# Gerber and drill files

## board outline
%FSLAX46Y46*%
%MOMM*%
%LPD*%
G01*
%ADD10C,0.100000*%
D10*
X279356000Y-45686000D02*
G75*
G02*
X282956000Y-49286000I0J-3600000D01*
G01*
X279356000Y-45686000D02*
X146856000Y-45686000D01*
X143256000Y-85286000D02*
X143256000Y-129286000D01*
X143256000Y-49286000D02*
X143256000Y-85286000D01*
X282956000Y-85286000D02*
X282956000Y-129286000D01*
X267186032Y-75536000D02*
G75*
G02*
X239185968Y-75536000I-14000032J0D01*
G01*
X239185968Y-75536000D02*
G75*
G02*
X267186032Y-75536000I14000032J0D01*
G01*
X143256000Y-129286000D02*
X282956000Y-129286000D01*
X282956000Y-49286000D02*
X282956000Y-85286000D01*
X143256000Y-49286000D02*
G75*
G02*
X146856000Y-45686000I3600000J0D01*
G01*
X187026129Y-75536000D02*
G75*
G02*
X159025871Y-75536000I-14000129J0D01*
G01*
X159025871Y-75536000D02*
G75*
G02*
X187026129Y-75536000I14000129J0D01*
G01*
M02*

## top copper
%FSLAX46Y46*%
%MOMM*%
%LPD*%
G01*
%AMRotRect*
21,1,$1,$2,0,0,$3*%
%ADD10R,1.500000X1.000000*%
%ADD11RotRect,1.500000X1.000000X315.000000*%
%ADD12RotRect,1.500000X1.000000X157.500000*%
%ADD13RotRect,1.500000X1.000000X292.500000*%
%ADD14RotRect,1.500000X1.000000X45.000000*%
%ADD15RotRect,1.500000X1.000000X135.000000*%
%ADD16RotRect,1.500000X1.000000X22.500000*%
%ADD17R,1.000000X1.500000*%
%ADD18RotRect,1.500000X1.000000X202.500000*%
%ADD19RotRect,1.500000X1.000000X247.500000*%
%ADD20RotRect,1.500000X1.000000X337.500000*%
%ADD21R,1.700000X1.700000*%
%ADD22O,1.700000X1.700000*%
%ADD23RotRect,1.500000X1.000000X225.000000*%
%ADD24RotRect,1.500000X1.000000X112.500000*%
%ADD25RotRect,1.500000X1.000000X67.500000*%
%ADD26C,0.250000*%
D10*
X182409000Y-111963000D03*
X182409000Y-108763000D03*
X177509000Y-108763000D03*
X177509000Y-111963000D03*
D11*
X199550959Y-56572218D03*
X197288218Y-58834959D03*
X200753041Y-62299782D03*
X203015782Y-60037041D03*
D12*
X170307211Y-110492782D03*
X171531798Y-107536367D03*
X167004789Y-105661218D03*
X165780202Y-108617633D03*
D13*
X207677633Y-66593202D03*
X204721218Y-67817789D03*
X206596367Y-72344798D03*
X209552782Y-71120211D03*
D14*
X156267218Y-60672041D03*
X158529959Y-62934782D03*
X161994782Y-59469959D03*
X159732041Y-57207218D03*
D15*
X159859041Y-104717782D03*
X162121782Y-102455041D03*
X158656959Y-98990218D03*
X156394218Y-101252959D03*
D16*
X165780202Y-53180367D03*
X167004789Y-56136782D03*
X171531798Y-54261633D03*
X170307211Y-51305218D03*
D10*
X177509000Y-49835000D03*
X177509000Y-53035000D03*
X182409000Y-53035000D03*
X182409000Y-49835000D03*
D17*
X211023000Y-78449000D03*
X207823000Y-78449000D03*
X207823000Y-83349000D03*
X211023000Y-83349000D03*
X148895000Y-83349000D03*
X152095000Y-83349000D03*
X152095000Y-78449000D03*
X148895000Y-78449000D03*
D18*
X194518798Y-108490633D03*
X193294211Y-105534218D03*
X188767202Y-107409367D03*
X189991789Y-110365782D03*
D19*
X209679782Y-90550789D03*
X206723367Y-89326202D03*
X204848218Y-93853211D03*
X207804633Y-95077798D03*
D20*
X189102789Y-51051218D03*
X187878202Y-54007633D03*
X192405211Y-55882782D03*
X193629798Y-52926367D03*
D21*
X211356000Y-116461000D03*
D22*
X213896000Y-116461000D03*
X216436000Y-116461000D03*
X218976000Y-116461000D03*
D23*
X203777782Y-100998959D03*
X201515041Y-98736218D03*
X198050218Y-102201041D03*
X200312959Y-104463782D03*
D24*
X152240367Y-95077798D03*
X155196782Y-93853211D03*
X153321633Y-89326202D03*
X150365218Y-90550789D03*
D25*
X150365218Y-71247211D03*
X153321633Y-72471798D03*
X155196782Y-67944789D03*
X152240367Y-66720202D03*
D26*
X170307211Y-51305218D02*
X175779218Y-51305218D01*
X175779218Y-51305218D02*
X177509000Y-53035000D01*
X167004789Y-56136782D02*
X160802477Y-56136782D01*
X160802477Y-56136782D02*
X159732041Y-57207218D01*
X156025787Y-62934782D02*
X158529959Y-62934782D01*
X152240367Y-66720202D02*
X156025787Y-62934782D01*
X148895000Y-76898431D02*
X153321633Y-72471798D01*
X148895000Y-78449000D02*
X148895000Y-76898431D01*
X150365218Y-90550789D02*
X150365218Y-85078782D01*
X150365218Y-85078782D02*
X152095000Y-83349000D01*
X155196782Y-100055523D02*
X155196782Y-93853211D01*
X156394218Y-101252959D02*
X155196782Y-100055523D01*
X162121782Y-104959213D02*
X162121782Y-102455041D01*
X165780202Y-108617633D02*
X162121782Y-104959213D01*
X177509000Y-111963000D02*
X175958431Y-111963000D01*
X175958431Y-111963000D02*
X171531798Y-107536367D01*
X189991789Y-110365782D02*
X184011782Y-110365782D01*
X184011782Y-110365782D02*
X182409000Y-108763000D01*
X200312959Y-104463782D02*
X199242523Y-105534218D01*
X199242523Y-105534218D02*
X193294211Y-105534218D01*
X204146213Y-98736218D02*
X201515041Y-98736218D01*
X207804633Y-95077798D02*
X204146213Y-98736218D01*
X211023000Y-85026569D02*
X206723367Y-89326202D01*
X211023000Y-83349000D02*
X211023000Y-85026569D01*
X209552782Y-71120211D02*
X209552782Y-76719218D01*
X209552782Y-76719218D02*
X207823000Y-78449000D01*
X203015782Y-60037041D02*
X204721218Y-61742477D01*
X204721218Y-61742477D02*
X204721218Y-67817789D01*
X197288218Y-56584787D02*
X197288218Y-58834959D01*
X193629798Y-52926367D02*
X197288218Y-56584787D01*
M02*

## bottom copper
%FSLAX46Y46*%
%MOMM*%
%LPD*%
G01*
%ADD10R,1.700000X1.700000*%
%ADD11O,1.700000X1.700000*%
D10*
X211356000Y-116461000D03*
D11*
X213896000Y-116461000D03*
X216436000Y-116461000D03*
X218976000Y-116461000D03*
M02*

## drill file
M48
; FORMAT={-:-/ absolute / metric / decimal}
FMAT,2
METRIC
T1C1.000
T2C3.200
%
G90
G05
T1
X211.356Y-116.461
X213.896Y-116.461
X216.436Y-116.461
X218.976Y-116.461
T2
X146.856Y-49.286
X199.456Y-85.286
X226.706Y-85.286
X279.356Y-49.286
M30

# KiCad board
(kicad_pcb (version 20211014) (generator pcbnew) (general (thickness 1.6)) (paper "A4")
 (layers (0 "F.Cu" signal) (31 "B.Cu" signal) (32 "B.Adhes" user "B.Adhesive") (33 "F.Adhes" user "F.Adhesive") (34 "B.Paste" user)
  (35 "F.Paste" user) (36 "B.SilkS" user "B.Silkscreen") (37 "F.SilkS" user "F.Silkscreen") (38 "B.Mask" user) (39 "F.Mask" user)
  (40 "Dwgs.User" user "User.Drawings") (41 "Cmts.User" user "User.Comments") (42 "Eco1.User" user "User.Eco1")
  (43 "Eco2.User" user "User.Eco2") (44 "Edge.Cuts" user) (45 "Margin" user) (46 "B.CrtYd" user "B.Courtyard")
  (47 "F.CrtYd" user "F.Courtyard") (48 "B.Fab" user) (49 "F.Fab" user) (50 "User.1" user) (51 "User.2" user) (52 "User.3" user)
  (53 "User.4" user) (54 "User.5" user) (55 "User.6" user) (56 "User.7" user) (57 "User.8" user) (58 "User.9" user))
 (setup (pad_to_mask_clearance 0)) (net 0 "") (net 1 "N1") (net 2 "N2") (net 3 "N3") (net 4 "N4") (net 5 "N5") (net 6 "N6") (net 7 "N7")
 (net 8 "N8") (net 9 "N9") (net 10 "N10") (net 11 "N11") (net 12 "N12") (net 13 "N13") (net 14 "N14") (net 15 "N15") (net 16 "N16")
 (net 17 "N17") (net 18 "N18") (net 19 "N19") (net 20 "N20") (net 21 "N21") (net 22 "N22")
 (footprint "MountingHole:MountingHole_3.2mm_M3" (layer "F.Cu") (at 226.706 85.286)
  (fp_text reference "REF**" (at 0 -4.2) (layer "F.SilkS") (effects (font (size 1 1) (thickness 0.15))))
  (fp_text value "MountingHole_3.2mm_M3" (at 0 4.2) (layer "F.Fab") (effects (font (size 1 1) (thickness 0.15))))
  (pad "" np_thru_hole circle locked (at 0 0) (size 3.2 3.2) (drill 3.2) (layers *.Cu *.Mask)))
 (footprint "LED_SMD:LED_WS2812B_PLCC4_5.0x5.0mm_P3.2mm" (layer "F.Cu") (at 179.959 110.363 180)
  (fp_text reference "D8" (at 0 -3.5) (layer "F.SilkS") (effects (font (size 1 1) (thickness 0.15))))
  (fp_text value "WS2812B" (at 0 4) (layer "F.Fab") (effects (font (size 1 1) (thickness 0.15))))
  (pad "1" smd rect locked (at -2.45 -1.6 180) (size 1.5 1) (layers "F.Cu" "F.Paste" "F.Mask") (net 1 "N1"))
  (pad "2" smd rect locked (at -2.45 1.6 180) (size 1.5 1) (layers "F.Cu" "F.Paste" "F.Mask") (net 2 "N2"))
  (pad "3" smd rect locked (at 2.45 1.6 180) (size 1.5 1) (layers "F.Cu" "F.Paste" "F.Mask") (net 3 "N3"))
  (pad "4" smd rect locked (at 2.45 -1.6 180) (size 1.5 1) (layers "F.Cu" "F.Paste" "F.Mask") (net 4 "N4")))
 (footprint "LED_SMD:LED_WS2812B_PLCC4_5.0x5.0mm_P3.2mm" (layer "F.Cu") (at 200.152 59.436 -45)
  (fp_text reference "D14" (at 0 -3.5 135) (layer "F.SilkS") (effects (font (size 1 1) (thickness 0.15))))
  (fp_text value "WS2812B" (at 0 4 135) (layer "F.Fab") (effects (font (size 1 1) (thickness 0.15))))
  (pad "1" smd rect locked (at -2.45 -1.6 315) (size 1.5 1) (layers "F.Cu" "F.Paste" "F.Mask") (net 1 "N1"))
  (pad "2" smd rect locked (at -2.45 1.6 315) (size 1.5 1) (layers "F.Cu" "F.Paste" "F.Mask") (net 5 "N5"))
  (pad "3" smd rect locked (at 2.45 1.6 315) (size 1.5 1) (layers "F.Cu" "F.Paste" "F.Mask") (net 3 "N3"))
  (pad "4" smd rect locked (at 2.45 -1.6 315) (size 1.5 1) (layers "F.Cu" "F.Paste" "F.Mask") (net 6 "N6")))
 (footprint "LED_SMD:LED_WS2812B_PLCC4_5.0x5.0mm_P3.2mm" (layer "F.Cu") (at 168.656 108.077 157.5)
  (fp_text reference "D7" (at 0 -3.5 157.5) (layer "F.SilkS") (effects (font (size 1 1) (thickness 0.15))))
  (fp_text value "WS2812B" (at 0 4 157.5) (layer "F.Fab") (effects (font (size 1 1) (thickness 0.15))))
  (pad "1" smd rect locked (at -2.45 -1.6 157.5) (size 1.5 1) (layers "F.Cu" "F.Paste" "F.Mask") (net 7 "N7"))
  (pad "2" smd rect locked (at -2.45 1.6 157.5) (size 1.5 1) (layers "F.Cu" "F.Paste" "F.Mask") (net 4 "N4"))
  (pad "3" smd rect locked (at 2.45 1.6 157.5) (size 1.5 1) (layers "F.Cu" "F.Paste" "F.Mask") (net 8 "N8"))
  (pad "4" smd rect locked (at 2.45 -1.6 157.5) (size 1.5 1) (layers "F.Cu" "F.Paste" "F.Mask") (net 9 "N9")))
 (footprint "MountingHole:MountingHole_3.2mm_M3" (layer "F.Cu") (at 279.356 49.286)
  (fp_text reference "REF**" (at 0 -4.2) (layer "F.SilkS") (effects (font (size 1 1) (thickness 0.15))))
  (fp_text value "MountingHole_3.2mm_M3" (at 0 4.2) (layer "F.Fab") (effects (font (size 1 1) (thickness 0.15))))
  (pad "" np_thru_hole circle locked (at 0 0) (size 3.2 3.2) (drill 3.2) (layers *.Cu *.Mask)))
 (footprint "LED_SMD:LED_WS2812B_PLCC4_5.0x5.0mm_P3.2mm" (layer "F.Cu") (at 207.137 69.469 -67.5)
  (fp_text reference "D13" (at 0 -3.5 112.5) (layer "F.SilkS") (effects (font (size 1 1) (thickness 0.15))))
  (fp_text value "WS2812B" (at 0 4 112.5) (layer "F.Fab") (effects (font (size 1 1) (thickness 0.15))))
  (pad "1" smd rect locked (at -2.45 -1.6 292.5) (size 1.5 1) (layers "F.Cu" "F.Paste" "F.Mask") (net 1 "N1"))
  (pad "2" smd rect locked (at -2.45 1.6 292.5) (size 1.5 1) (layers "F.Cu" "F.Paste" "F.Mask") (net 6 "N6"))
  (pad "3" smd rect locked (at 2.45 1.6 292.5) (size 1.5 1) (layers "F.Cu" "F.Paste" "F.Mask") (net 3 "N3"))
  (pad "4" smd rect locked (at 2.45 -1.6 292.5) (size 1.5 1) (layers "F.Cu" "F.Paste" "F.Mask") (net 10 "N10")))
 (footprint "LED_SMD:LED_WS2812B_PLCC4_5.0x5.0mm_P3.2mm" (layer "F.Cu") (at 159.131 60.071 45)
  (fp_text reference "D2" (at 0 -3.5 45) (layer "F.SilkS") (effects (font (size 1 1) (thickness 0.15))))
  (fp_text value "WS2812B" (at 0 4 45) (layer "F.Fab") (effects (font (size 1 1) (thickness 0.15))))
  (pad "1" smd rect locked (at -2.45 -1.6 45) (size 1.5 1) (layers "F.Cu" "F.Paste" "F.Mask") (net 7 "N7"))
  (pad "2" smd rect locked (at -2.45 1.6 45) (size 1.5 1) (layers "F.Cu" "F.Paste" "F.Mask") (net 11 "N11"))
  (pad "3" smd rect locked (at 2.45 1.6 45) (size 1.5 1) (layers "F.Cu" "F.Paste" "F.Mask") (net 8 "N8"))
  (pad "4" smd rect locked (at 2.45 -1.6 45) (size 1.5 1) (layers "F.Cu" "F.Paste" "F.Mask") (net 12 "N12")))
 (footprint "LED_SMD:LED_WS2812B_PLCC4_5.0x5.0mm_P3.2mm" (layer "F.Cu") (at 159.258 101.854 135)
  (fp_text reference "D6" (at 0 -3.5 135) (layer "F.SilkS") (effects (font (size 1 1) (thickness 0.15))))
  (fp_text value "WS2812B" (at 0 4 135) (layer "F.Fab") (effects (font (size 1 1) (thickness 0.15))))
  (pad "1" smd rect locked (at -2.45 -1.6 135) (size 1.5 1) (layers "F.Cu" "F.Paste" "F.Mask") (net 7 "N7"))
  (pad "2" smd rect locked (at -2.45 1.6 135) (size 1.5 1) (layers "F.Cu" "F.Paste" "F.Mask") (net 9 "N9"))
  (pad "3" smd rect locked (at 2.45 1.6 135) (size 1.5 1) (layers "F.Cu" "F.Paste" "F.Mask") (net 8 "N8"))
  (pad "4" smd rect locked (at 2.45 -1.6 135) (size 1.5 1) (layers "F.Cu" "F.Paste" "F.Mask") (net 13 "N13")))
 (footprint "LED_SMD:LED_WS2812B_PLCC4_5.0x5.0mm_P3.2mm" (layer "F.Cu") (at 168.656 53.721 22.5)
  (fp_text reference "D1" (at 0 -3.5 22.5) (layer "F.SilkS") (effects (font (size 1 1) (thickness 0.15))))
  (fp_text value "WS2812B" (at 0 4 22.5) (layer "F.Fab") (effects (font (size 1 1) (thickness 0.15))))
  (pad "1" smd rect locked (at -2.45 -1.6 22.5) (size 1.5 1) (layers "F.Cu" "F.Paste" "F.Mask") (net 7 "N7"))
  (pad "2" smd rect locked (at -2.45 1.6 22.5) (size 1.5 1) (layers "F.Cu" "F.Paste" "F.Mask") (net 12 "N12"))
  (pad "3" smd rect locked (at 2.45 1.6 22.5) (size 1.5 1) (layers "F.Cu" "F.Paste" "F.Mask") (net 8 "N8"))
  (pad "4" smd rect locked (at 2.45 -1.6 22.5) (size 1.5 1) (layers "F.Cu" "F.Paste" "F.Mask") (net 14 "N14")))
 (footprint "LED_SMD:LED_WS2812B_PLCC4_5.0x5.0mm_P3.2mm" (layer "F.Cu") (at 179.959 51.435)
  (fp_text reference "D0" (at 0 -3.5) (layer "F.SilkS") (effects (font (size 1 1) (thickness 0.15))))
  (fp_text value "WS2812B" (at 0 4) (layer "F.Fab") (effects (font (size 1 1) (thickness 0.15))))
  (pad "1" smd rect locked (at -2.45 -1.6) (size 1.5 1) (layers "F.Cu" "F.Paste" "F.Mask") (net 7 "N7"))
  (pad "2" smd rect locked (at -2.45 1.6) (size 1.5 1) (layers "F.Cu" "F.Paste" "F.Mask") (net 14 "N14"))
  (pad "3" smd rect locked (at 2.45 1.6) (size 1.5 1) (layers "F.Cu" "F.Paste" "F.Mask") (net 8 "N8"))
  (pad "4" smd rect locked (at 2.45 -1.6) (size 1.5 1) (layers "F.Cu" "F.Paste" "F.Mask") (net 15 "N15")))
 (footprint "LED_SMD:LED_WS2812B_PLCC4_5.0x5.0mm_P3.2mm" (layer "F.Cu") (at 209.423 80.899 -90)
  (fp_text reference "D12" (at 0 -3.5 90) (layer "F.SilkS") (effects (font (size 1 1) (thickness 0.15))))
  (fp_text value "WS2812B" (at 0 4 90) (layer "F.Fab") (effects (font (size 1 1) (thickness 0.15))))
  (pad "1" smd rect locked (at -2.45 -1.6 270) (size 1.5 1) (layers "F.Cu" "F.Paste" "F.Mask") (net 1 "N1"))
  (pad "2" smd rect locked (at -2.45 1.6 270) (size 1.5 1) (layers "F.Cu" "F.Paste" "F.Mask") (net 10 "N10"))
  (pad "3" smd rect locked (at 2.45 1.6 270) (size 1.5 1) (layers "F.Cu" "F.Paste" "F.Mask") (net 3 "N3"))
  (pad "4" smd rect locked (at 2.45 -1.6 270) (size 1.5 1) (layers "F.Cu" "F.Paste" "F.Mask") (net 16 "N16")))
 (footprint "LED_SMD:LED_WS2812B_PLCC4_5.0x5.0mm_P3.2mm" (layer "F.Cu") (at 150.495 80.899 90)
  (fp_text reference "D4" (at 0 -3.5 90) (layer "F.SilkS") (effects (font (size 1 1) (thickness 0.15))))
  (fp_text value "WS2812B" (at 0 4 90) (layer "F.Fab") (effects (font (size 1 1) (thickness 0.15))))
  (pad "1" smd rect locked (at -2.45 -1.6 90) (size 1.5 1) (layers "F.Cu" "F.Paste" "F.Mask") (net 7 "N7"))
  (pad "2" smd rect locked (at -2.45 1.6 90) (size 1.5 1) (layers "F.Cu" "F.Paste" "F.Mask") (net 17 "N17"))
  (pad "3" smd rect locked (at 2.45 1.6 90) (size 1.5 1) (layers "F.Cu" "F.Paste" "F.Mask") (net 8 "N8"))
  (pad "4" smd rect locked (at 2.45 -1.6 90) (size 1.5 1) (layers "F.Cu" "F.Paste" "F.Mask") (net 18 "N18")))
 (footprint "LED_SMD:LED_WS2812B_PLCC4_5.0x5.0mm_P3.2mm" (layer "F.Cu") (at 191.643 107.95 -157.5)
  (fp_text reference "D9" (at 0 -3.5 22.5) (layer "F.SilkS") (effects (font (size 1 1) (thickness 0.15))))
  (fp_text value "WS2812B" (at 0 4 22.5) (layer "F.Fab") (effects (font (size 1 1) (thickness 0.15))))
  (pad "1" smd rect locked (at -2.45 -1.6 202.5) (size 1.5 1) (layers "F.Cu" "F.Paste" "F.Mask") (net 1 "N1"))
  (pad "2" smd rect locked (at -2.45 1.6 202.5) (size 1.5 1) (layers "F.Cu" "F.Paste" "F.Mask") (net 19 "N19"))
  (pad "3" smd rect locked (at 2.45 1.6 202.5) (size 1.5 1) (layers "F.Cu" "F.Paste" "F.Mask") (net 3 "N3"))
  (pad "4" smd rect locked (at 2.45 -1.6 202.5) (size 1.5 1) (layers "F.Cu" "F.Paste" "F.Mask") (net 2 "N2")))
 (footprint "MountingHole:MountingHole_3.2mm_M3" (layer "F.Cu") (at 146.856 49.286)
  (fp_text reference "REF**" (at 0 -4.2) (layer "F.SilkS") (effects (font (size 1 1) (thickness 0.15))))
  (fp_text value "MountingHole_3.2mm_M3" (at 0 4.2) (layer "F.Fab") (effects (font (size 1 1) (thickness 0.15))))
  (pad "" np_thru_hole circle locked (at 0 0) (size 3.2 3.2) (drill 3.2) (layers *.Cu *.Mask)))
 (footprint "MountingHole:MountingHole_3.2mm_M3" (layer "F.Cu") (at 199.456 85.286)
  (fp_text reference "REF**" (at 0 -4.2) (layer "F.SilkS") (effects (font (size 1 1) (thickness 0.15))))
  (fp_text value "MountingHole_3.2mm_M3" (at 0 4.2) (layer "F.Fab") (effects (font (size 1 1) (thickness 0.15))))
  (pad "" np_thru_hole circle locked (at 0 0) (size 3.2 3.2) (drill 3.2) (layers *.Cu *.Mask)))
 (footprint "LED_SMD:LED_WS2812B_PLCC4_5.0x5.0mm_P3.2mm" (layer "F.Cu") (at 207.264 92.202 -112.5)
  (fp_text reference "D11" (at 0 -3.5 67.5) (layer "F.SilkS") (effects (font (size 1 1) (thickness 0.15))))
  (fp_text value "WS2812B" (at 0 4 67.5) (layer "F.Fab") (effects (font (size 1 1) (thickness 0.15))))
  (pad "1" smd rect locked (at -2.45 -1.6 247.5) (size 1.5 1) (layers "F.Cu" "F.Paste" "F.Mask") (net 1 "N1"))
  (pad "2" smd rect locked (at -2.45 1.6 247.5) (size 1.5 1) (layers "F.Cu" "F.Paste" "F.Mask") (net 16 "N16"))
  (pad "3" smd rect locked (at 2.45 1.6 247.5) (size 1.5 1) (layers "F.Cu" "F.Paste" "F.Mask") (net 3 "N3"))
  (pad "4" smd rect locked (at 2.45 -1.6 247.5) (size 1.5 1) (layers "F.Cu" "F.Paste" "F.Mask") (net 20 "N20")))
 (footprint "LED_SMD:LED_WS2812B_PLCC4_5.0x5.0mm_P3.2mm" (layer "F.Cu") (at 190.754 53.467 -22.5)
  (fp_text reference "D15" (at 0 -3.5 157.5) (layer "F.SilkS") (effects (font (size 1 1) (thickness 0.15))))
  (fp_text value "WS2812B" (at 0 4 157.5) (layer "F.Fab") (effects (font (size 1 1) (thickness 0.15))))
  (pad "1" smd rect locked (at -2.45 -1.6 337.5) (size 1.5 1) (layers "F.Cu" "F.Paste" "F.Mask") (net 1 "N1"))
  (pad "2" smd rect locked (at -2.45 1.6 337.5) (size 1.5 1) (layers "F.Cu" "F.Paste" "F.Mask") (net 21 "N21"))
  (pad "3" smd rect locked (at 2.45 1.6 337.5) (size 1.5 1) (layers "F.Cu" "F.Paste" "F.Mask") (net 3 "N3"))
  (pad "4" smd rect locked (at 2.45 -1.6 337.5) (size 1.5 1) (layers "F.Cu" "F.Paste" "F.Mask") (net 5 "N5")))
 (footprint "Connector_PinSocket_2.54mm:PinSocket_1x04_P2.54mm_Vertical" (layer "F.Cu") (at 211.356 116.461 90)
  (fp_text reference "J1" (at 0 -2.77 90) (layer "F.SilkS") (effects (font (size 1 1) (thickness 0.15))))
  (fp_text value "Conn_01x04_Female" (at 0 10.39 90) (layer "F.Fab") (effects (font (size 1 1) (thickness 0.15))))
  (pad "1" thru_hole rect locked (at 0 0 90) (size 1.7 1.7) (drill 1) (layers *.Cu *.Mask) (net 8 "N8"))
  (pad "2" thru_hole oval locked (at 0 2.54 90) (size 1.7 1.7) (drill 1) (layers *.Cu *.Mask) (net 7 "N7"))
  (pad "3" thru_hole oval locked (at 0 5.08 90) (size 1.7 1.7) (drill 1) (layers *.Cu *.Mask) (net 15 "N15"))
  (pad "4" thru_hole oval locked (at 0 7.62 90) (size 1.7 1.7) (drill 1) (layers *.Cu *.Mask) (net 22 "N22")))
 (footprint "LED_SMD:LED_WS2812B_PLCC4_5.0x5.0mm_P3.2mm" (layer "F.Cu") (at 200.914 101.6 -135)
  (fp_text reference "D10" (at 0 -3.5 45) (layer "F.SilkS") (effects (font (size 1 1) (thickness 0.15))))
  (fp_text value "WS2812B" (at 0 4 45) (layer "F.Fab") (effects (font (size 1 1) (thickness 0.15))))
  (pad "1" smd rect locked (at -2.45 -1.6 225) (size 1.5 1) (layers "F.Cu" "F.Paste" "F.Mask") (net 1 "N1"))
  (pad "2" smd rect locked (at -2.45 1.6 225) (size 1.5 1) (layers "F.Cu" "F.Paste" "F.Mask") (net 20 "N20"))
  (pad "3" smd rect locked (at 2.45 1.6 225) (size 1.5 1) (layers "F.Cu" "F.Paste" "F.Mask") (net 3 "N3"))
  (pad "4" smd rect locked (at 2.45 -1.6 225) (size 1.5 1) (layers "F.Cu" "F.Paste" "F.Mask") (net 19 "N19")))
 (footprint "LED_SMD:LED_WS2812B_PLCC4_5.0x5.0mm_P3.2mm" (layer "F.Cu") (at 152.781 92.202 112.5)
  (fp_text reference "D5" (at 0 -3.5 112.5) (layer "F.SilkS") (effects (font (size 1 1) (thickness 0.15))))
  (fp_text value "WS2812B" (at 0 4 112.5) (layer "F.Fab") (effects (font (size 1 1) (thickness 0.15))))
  (pad "1" smd rect locked (at -2.45 -1.6 112.5) (size 1.5 1) (layers "F.Cu" "F.Paste" "F.Mask") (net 7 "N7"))
  (pad "2" smd rect locked (at -2.45 1.6 112.5) (size 1.5 1) (layers "F.Cu" "F.Paste" "F.Mask") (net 13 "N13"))
  (pad "3" smd rect locked (at 2.45 1.6 112.5) (size 1.5 1) (layers "F.Cu" "F.Paste" "F.Mask") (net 8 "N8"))
  (pad "4" smd rect locked (at 2.45 -1.6 112.5) (size 1.5 1) (layers "F.Cu" "F.Paste" "F.Mask") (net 17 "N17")))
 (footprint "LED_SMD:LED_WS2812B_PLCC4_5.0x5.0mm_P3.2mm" (layer "F.Cu") (at 152.781 69.596 67.5)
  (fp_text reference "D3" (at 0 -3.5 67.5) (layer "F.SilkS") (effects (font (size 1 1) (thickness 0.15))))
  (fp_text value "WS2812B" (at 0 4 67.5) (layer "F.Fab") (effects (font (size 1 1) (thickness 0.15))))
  (pad "1" smd rect locked (at -2.45 -1.6 67.5) (size 1.5 1) (layers "F.Cu" "F.Paste" "F.Mask") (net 7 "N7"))
  (pad "2" smd rect locked (at -2.45 1.6 67.5) (size 1.5 1) (layers "F.Cu" "F.Paste" "F.Mask") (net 18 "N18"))
  (pad "3" smd rect locked (at 2.45 1.6 67.5) (size 1.5 1) (layers "F.Cu" "F.Paste" "F.Mask") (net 8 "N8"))
  (pad "4" smd rect locked (at 2.45 -1.6 67.5) (size 1.5 1) (layers "F.Cu" "F.Paste" "F.Mask") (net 11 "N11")))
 (gr_arc (start 279.356 45.686) (mid 281.901584 46.740416) (end 282.956 49.286) (layer "Edge.Cuts") (width 0.1))
 (gr_line (start 279.356 45.686) (end 146.856 45.686) (layer "Edge.Cuts") (width 0.1))
 (gr_line (start 143.256 85.286) (end 143.256 129.286) (layer "Edge.Cuts") (width 0.1))
 (gr_line (start 143.256 49.286) (end 143.256 85.286) (layer "Edge.Cuts") (width 0.1))
 (gr_line (start 282.956 85.286) (end 282.956 129.286) (layer "Edge.Cuts") (width 0.1))
 (gr_circle (center 253.186 75.536) (end 253.216 89.536) (layer "Edge.Cuts") (width 0.1) (fill none))
 (gr_line (start 143.256 129.286) (end 282.956 129.286) (layer "Edge.Cuts") (width 0.1))
 (gr_line (start 282.956 49.286) (end 282.956 85.286) (layer "Edge.Cuts") (width 0.1))
 (gr_arc (start 143.256 49.286) (mid 144.310416 46.740416) (end 146.856 45.686) (layer "Edge.Cuts") (width 0.1))
 (gr_circle (center 173.026 75.536) (end 172.966 89.536) (layer "Edge.Cuts") (width 0.1) (fill none))
 (segment (start 170.307211 51.305218) (end 175.779218 51.305218) (width 0.25) (layer "F.Cu") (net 14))
 (segment (start 175.779218 51.305218) (end 177.509 53.035) (width 0.25) (layer "F.Cu") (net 14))
 (segment (start 167.004789 56.136782) (end 160.802477 56.136782) (width 0.25) (layer "F.Cu") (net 12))
 (segment (start 160.802477 56.136782) (end 159.732041 57.207218) (width 0.25) (layer "F.Cu") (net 12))
 (segment (start 156.025787 62.934782) (end 158.529959 62.934782) (width 0.25) (layer "F.Cu") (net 11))
 (segment (start 152.240367 66.720202) (end 156.025787 62.934782) (width 0.25) (layer "F.Cu") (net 11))
 (segment (start 148.895 76.898431) (end 153.321633 72.471798) (width 0.25) (layer "F.Cu") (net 18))
 (segment (start 148.895 78.449) (end 148.895 76.898431) (width 0.25) (layer "F.Cu") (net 18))
 (segment (start 150.365218 90.550789) (end 150.365218 85.078782) (width 0.25) (layer "F.Cu") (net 17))
 (segment (start 150.365218 85.078782) (end 152.095 83.349) (width 0.25) (layer "F.Cu") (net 17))
 (segment (start 155.196782 100.055523) (end 155.196782 93.853211) (width 0.25) (layer "F.Cu") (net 13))
 (segment (start 156.394218 101.252959) (end 155.196782 100.055523) (width 0.25) (layer "F.Cu") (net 13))
 (segment (start 162.121782 104.959213) (end 162.121782 102.455041) (width 0.25) (layer "F.Cu") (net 9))
 (segment (start 165.780202 108.617633) (end 162.121782 104.959213) (width 0.25) (layer "F.Cu") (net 9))
 (segment (start 177.509 111.963) (end 175.958431 111.963) (width 0.25) (layer "F.Cu") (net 4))
 (segment (start 175.958431 111.963) (end 171.531798 107.536367) (width 0.25) (layer "F.Cu") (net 4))
 (segment (start 189.991789 110.365782) (end 184.011782 110.365782) (width 0.25) (layer "F.Cu") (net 2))
 (segment (start 184.011782 110.365782) (end 182.409 108.763) (width 0.25) (layer "F.Cu") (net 2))
 (segment (start 200.312959 104.463782) (end 199.242523 105.534218) (width 0.25) (layer "F.Cu") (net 19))
 (segment (start 199.242523 105.534218) (end 193.294211 105.534218) (width 0.25) (layer "F.Cu") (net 19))
 (segment (start 204.146213 98.736218) (end 201.515041 98.736218) (width 0.25) (layer "F.Cu") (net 20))
 (segment (start 207.804633 95.077798) (end 204.146213 98.736218) (width 0.25) (layer "F.Cu") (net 20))
 (segment (start 211.023 85.026569) (end 206.723367 89.326202) (width 0.25) (layer "F.Cu") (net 16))
 (segment (start 211.023 83.349) (end 211.023 85.026569) (width 0.25) (layer "F.Cu") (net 16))
 (segment (start 209.552782 71.120211) (end 209.552782 76.719218) (width 0.25) (layer "F.Cu") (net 10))
 (segment (start 209.552782 76.719218) (end 207.823 78.449) (width 0.25) (layer "F.Cu") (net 10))
 (segment (start 203.015782 60.037041) (end 204.721218 61.742477) (width 0.25) (layer "F.Cu") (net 6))
 (segment (start 204.721218 61.742477) (end 204.721218 67.817789) (width 0.25) (layer "F.Cu") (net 6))
 (segment (start 197.288218 56.584787) (end 197.288218 58.834959) (width 0.25) (layer "F.Cu") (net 5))
 (segment (start 193.629798 52.926367) (end 197.288218 56.584787) (width 0.25) (layer "F.Cu") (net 5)))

